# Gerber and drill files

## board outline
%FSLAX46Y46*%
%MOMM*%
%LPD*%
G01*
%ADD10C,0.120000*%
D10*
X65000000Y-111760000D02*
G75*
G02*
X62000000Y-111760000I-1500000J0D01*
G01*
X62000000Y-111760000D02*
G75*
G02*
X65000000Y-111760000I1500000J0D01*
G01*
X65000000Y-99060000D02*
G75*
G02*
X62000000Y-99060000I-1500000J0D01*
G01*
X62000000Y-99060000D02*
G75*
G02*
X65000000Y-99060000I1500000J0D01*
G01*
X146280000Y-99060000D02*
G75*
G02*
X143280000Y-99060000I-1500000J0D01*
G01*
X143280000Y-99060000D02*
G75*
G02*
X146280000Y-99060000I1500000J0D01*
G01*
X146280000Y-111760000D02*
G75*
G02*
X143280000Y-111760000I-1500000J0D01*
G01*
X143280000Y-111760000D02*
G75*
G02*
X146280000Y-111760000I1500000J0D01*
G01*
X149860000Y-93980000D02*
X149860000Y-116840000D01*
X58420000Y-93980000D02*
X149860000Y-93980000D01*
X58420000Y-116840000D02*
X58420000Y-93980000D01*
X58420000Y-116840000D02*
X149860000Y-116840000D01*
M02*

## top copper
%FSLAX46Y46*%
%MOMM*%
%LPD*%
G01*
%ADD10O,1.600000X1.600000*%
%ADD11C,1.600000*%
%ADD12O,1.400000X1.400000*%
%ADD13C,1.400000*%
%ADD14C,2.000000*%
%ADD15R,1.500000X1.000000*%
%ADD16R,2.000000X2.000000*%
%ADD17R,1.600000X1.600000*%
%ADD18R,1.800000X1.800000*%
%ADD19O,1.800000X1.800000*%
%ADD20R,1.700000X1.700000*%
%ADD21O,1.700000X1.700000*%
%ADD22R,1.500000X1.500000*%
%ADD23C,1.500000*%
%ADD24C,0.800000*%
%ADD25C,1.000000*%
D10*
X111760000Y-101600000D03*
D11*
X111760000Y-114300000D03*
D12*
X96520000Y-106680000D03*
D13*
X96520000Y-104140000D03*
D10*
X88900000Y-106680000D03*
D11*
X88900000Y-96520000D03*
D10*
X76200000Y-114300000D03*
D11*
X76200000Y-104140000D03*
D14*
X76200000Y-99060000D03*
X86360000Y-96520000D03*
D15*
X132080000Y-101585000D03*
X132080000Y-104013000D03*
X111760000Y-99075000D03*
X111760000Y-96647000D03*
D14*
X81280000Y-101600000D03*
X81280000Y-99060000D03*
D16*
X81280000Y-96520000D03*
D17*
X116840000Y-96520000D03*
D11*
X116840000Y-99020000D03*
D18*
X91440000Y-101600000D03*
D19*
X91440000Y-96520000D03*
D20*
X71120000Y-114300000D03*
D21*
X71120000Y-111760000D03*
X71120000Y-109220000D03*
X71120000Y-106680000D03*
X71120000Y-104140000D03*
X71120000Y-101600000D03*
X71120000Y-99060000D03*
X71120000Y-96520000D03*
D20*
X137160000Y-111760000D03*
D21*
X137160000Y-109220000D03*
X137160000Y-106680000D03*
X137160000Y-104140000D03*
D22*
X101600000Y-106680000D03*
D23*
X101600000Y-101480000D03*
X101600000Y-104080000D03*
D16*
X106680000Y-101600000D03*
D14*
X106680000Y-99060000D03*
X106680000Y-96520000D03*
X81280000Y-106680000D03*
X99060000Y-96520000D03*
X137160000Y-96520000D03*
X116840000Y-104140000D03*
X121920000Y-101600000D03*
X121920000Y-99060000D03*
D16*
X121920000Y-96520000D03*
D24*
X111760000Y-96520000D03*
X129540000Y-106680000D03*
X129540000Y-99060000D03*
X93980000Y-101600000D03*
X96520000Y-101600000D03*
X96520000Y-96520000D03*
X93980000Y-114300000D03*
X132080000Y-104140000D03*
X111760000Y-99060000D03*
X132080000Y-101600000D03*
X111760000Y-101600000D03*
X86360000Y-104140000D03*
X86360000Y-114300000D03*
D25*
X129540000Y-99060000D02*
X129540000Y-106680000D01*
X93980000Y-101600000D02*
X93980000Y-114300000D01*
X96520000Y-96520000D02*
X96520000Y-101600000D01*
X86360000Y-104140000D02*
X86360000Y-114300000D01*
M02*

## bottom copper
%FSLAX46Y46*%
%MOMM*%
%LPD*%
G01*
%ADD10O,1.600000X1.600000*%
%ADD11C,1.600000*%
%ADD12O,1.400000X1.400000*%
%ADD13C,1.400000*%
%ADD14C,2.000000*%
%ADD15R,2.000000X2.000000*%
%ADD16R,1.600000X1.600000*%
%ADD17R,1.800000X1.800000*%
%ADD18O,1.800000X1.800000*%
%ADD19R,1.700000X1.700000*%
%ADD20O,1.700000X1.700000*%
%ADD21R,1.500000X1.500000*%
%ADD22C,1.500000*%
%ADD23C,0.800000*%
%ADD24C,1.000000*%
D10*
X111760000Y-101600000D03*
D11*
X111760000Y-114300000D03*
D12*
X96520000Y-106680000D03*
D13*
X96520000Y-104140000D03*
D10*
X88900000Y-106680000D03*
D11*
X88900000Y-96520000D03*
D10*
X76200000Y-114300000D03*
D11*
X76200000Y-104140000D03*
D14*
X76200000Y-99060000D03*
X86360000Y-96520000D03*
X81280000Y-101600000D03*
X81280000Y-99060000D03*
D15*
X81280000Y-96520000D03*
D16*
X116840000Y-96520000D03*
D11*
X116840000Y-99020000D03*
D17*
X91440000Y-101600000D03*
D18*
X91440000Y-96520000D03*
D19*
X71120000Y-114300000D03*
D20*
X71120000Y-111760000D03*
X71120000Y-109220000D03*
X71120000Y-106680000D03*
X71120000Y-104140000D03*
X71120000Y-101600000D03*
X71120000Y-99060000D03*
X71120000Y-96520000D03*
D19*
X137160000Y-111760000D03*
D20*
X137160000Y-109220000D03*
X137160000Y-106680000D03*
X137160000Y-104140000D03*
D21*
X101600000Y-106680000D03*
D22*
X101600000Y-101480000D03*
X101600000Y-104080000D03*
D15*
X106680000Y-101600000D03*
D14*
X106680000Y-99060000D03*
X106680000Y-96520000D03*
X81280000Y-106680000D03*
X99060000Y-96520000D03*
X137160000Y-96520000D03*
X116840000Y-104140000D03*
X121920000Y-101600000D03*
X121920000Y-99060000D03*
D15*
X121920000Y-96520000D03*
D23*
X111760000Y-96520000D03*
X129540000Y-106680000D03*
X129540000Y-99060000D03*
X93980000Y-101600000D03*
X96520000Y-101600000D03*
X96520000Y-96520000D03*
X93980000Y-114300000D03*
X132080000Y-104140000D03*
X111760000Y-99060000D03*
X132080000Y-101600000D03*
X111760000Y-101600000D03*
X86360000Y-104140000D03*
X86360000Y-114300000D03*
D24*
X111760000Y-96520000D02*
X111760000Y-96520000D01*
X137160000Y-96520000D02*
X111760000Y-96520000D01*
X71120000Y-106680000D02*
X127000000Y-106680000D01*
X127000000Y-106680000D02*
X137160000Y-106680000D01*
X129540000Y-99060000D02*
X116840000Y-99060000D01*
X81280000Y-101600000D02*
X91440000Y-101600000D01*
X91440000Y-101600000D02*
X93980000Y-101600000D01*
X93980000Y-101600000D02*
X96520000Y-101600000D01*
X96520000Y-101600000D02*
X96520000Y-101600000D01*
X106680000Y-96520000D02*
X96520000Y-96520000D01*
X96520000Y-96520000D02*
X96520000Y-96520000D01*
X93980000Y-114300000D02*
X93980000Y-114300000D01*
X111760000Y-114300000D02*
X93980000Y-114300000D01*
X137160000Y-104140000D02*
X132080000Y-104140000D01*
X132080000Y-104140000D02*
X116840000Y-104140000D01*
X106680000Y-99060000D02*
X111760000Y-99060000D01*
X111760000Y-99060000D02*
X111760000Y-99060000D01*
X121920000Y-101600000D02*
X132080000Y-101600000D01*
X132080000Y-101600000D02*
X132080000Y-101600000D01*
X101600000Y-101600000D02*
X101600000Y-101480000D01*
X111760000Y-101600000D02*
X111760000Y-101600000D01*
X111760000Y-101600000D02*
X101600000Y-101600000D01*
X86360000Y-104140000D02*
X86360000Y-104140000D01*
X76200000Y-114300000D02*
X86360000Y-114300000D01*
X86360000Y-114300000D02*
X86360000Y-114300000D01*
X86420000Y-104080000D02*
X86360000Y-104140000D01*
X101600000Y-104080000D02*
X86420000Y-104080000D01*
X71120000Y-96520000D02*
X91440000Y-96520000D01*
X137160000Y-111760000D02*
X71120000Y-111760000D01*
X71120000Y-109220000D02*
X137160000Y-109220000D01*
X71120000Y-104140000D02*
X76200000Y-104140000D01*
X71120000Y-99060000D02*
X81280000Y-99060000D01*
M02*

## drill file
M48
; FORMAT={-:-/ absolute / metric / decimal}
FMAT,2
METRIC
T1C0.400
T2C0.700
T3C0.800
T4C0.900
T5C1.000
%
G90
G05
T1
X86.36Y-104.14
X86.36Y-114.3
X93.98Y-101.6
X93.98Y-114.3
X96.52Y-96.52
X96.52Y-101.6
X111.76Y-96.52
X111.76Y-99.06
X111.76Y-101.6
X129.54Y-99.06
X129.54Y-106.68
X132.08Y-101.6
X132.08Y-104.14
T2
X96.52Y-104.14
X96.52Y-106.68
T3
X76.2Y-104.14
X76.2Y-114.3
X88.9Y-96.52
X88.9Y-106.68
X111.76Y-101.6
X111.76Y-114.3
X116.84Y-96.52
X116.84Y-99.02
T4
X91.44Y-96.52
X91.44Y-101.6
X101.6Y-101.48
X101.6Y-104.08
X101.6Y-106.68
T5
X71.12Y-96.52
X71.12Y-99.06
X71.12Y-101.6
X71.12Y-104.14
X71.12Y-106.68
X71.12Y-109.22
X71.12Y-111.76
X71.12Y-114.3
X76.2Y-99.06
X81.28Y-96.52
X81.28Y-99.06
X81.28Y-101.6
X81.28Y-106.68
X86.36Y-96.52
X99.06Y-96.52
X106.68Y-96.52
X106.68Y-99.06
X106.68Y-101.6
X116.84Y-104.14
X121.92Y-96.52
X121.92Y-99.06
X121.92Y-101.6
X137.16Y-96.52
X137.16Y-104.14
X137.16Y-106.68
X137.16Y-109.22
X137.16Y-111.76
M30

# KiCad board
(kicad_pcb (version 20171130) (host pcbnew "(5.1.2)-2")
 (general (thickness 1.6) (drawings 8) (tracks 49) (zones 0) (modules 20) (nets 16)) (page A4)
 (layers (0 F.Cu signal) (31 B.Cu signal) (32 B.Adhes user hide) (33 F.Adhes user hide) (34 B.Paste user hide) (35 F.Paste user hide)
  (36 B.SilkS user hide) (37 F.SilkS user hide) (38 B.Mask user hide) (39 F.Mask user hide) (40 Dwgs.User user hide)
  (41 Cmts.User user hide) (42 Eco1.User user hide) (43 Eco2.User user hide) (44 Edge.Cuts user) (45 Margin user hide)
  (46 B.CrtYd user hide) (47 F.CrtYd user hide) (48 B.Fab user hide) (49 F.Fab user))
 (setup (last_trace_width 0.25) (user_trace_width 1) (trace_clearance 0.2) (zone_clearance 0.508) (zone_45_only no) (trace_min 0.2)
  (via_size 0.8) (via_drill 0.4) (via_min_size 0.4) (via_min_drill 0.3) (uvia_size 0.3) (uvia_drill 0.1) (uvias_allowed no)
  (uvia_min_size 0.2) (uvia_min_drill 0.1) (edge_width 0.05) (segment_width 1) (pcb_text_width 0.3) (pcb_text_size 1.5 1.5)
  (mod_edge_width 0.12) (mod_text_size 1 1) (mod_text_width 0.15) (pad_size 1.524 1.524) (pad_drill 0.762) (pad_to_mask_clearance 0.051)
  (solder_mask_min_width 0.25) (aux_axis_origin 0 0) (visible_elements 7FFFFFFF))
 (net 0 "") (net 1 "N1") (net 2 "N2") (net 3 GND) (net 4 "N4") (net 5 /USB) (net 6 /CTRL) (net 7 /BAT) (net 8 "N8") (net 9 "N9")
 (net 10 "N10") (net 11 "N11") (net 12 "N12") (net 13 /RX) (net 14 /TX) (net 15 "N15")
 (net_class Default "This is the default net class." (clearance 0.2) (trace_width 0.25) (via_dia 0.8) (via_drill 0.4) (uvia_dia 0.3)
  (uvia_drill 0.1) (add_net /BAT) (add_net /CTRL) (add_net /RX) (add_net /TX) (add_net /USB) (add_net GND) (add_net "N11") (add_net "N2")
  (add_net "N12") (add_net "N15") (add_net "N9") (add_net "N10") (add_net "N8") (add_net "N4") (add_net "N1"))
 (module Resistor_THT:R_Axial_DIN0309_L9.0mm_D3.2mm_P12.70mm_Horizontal (layer F.Cu) (at 111.76 114.3 90)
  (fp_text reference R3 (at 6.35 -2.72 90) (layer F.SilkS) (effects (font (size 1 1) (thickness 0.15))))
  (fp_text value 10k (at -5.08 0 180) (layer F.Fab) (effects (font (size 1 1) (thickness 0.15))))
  (pad 2 thru_hole oval (at 12.7 0 90) (size 1.6 1.6) (drill 0.8) (layers *.Cu *.Mask) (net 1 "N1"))
  (pad 1 thru_hole circle (at 0 0 90) (size 1.6 1.6) (drill 0.8) (layers *.Cu *.Mask) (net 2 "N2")))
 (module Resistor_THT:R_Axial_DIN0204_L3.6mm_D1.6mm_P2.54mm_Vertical (layer F.Cu) (at 96.52 104.14 270)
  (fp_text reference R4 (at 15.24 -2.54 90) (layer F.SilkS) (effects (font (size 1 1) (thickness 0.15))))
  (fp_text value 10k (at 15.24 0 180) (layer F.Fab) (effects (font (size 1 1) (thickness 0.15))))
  (pad 2 thru_hole oval (at 2.54 0 270) (size 1.4 1.4) (drill 0.7) (layers *.Cu *.Mask) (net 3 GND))
  (pad 1 thru_hole circle (at 0 0 270) (size 1.4 1.4) (drill 0.7) (layers *.Cu *.Mask) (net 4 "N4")))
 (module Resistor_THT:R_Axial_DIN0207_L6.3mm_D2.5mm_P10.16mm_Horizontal (layer F.Cu) (at 88.9 96.52 270)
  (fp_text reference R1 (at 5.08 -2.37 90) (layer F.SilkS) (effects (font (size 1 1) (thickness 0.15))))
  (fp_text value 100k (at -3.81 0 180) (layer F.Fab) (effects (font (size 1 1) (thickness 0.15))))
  (pad 2 thru_hole oval (at 10.16 0 270) (size 1.6 1.6) (drill 0.8) (layers *.Cu *.Mask) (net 3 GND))
  (pad 1 thru_hole circle (at 0 0 270) (size 1.6 1.6) (drill 0.8) (layers *.Cu *.Mask) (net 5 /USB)))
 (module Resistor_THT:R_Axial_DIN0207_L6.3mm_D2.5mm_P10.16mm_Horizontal (layer F.Cu) (at 76.2 104.14 270)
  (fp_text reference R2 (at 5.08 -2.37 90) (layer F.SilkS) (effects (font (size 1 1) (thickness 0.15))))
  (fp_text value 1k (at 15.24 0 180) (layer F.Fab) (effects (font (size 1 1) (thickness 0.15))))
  (pad 2 thru_hole oval (at 10.16 0 270) (size 1.6 1.6) (drill 0.8) (layers *.Cu *.Mask) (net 4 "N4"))
  (pad 1 thru_hole circle (at 0 0 270) (size 1.6 1.6) (drill 0.8) (layers *.Cu *.Mask) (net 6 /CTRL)))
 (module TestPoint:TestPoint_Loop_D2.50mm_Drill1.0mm (layer F.Cu) (at 76.2 99.06)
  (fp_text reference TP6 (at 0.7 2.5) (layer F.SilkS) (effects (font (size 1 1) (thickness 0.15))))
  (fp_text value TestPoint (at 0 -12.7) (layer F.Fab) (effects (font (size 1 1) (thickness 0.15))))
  (pad 1 thru_hole circle (at 0 0) (size 2 2) (drill 1) (layers *.Cu *.Mask) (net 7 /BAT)))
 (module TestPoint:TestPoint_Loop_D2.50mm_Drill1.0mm (layer F.Cu) (at 86.36 96.52)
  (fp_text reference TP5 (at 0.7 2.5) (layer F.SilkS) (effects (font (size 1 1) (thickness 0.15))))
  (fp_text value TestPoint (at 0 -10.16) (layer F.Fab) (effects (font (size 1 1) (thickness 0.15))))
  (pad 1 thru_hole circle (at 0 0) (size 2 2) (drill 1) (layers *.Cu *.Mask) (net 5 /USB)))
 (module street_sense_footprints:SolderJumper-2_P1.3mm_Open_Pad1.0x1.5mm (layer F.Cu) (at 132.08 101.6 270)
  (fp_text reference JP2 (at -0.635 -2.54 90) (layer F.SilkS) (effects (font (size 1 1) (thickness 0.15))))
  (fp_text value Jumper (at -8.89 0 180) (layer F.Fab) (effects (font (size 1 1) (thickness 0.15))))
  (pad 1 smd rect (at -0.015 0 270) (size 1 1.5) (layers F.Cu F.Mask) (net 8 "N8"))
  (pad 2 smd rect (at 2.413 0 270) (size 1 1.5) (layers F.Cu F.Mask) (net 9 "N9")))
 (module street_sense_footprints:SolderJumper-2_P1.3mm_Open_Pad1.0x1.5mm (layer F.Cu) (at 111.76 99.06 90)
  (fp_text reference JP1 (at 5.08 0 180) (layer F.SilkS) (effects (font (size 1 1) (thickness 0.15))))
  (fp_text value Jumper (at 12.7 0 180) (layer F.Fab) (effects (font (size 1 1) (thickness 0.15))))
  (pad 1 smd rect (at -0.015 0 90) (size 1 1.5) (layers F.Cu F.Mask) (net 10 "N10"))
  (pad 2 smd rect (at 2.413 0 90) (size 1 1.5) (layers F.Cu F.Mask) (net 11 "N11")))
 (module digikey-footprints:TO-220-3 (layer F.Cu) (at 81.28 96.52 270)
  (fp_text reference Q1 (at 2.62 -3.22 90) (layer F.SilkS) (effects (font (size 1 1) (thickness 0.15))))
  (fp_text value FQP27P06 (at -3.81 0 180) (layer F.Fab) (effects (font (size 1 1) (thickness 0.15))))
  (pad 3 thru_hole circle (at 5.08 0 270) (size 2 2) (drill 1) (layers *.Cu *.Mask) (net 2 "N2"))
  (pad 2 thru_hole circle (at 2.54 0 270) (size 2 2) (drill 1) (layers *.Cu *.Mask) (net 7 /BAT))
  (pad 1 thru_hole rect (at 0 0 270) (size 2 2) (drill 1) (layers *.Cu *.Mask) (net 5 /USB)))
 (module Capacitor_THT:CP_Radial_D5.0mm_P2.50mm (layer F.Cu) (at 116.84 96.52 270)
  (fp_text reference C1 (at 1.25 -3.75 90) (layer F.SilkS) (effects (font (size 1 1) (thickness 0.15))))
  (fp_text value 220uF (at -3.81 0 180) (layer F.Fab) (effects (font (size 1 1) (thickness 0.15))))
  (pad 1 thru_hole rect (at 0 0 270) (size 1.6 1.6) (drill 0.8) (layers *.Cu *.Mask) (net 11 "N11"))
  (pad 2 thru_hole circle (at 2.5 0 270) (size 1.6 1.6) (drill 0.8) (layers *.Cu *.Mask) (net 3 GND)))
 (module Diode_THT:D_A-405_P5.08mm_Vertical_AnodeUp (layer F.Cu) (at 91.44 101.6 90)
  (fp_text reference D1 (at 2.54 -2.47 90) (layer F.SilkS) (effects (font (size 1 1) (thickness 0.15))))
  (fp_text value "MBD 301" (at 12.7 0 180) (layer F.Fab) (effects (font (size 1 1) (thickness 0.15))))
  (pad 1 thru_hole rect (at 0 0 90) (size 1.8 1.8) (drill 0.9) (layers *.Cu *.Mask) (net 2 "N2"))
  (pad 2 thru_hole oval (at 5.08 0 90) (size 1.8 1.8) (drill 0.9) (layers *.Cu *.Mask) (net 5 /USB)))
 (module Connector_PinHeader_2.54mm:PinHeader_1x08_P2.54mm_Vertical (layer F.Cu) (at 71.12 114.3 180)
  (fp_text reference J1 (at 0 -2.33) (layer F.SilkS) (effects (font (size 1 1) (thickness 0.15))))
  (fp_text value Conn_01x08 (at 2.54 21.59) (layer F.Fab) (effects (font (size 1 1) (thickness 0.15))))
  (pad 1 thru_hole rect (at 0 0 180) (size 1.7 1.7) (drill 1) (layers *.Cu *.Mask) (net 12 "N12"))
  (pad 2 thru_hole oval (at 0 2.54 180) (size 1.7 1.7) (drill 1) (layers *.Cu *.Mask) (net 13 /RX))
  (pad 3 thru_hole oval (at 0 5.08 180) (size 1.7 1.7) (drill 1) (layers *.Cu *.Mask) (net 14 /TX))
  (pad 4 thru_hole oval (at 0 7.62 180) (size 1.7 1.7) (drill 1) (layers *.Cu *.Mask) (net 3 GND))
  (pad 5 thru_hole oval (at 0 10.16 180) (size 1.7 1.7) (drill 1) (layers *.Cu *.Mask) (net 6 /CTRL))
  (pad 6 thru_hole oval (at 0 12.7 180) (size 1.7 1.7) (drill 1) (layers *.Cu *.Mask) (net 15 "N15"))
  (pad 7 thru_hole oval (at 0 15.24 180) (size 1.7 1.7) (drill 1) (layers *.Cu *.Mask) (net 7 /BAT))
  (pad 8 thru_hole oval (at 0 17.78 180) (size 1.7 1.7) (drill 1) (layers *.Cu *.Mask) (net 5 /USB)))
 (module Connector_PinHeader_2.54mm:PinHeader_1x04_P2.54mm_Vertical (layer F.Cu) (at 137.16 111.76 180)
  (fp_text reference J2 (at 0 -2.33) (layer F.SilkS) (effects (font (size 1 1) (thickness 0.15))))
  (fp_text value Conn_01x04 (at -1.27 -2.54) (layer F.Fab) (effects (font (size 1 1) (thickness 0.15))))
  (pad 1 thru_hole rect (at 0 0 180) (size 1.7 1.7) (drill 1) (layers *.Cu *.Mask) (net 13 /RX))
  (pad 2 thru_hole oval (at 0 2.54 180) (size 1.7 1.7) (drill 1) (layers *.Cu *.Mask) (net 14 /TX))
  (pad 3 thru_hole oval (at 0 5.08 180) (size 1.7 1.7) (drill 1) (layers *.Cu *.Mask) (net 3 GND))
  (pad 4 thru_hole oval (at 0 7.62 180) (size 1.7 1.7) (drill 1) (layers *.Cu *.Mask) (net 9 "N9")))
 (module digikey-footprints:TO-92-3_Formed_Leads (layer F.Cu) (at 101.6 106.68 90)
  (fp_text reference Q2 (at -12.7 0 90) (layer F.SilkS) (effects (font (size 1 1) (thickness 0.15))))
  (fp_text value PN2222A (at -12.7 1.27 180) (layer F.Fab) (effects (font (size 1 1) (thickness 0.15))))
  (pad 1 thru_hole rect (at 0 0 270) (size 1.5 1.5) (drill 0.9) (layers *.Cu *.Mask) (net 3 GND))
  (pad 3 thru_hole circle (at 5.2 0 270) (size 1.5 1.5) (drill 0.9) (layers *.Cu *.Mask) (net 1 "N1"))
  (pad 2 thru_hole circle (at 2.6 0 270) (size 1.5 1.5) (drill 0.9) (layers *.Cu *.Mask) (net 4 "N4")))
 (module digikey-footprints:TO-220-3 (layer F.Cu) (at 106.68 101.6 90)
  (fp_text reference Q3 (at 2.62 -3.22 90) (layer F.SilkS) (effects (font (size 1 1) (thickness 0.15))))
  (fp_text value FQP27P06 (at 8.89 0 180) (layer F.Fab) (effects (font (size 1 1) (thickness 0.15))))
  (pad 1 thru_hole rect (at 0 0 90) (size 2 2) (drill 1) (layers *.Cu *.Mask) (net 1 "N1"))
  (pad 2 thru_hole circle (at 2.54 0 90) (size 2 2) (drill 1) (layers *.Cu *.Mask) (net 10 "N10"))
  (pad 3 thru_hole circle (at 5.08 0 90) (size 2 2) (drill 1) (layers *.Cu *.Mask) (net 2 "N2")))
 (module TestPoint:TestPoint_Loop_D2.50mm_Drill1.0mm (layer F.Cu) (at 81.28 106.68)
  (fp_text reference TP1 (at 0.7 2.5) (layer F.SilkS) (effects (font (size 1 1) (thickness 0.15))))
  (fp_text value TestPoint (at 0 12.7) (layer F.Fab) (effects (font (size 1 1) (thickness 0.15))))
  (pad 1 thru_hole circle (at 0 0) (size 2 2) (drill 1) (layers *.Cu *.Mask) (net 3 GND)))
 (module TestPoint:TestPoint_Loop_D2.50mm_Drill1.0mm (layer F.Cu) (at 99.06 96.52)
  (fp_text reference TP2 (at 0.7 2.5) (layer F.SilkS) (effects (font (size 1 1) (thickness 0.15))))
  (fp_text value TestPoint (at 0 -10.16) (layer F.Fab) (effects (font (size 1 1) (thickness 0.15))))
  (pad 1 thru_hole circle (at 0 0) (size 2 2) (drill 1) (layers *.Cu *.Mask) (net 2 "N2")))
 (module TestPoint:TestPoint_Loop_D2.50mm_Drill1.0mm (layer F.Cu) (at 137.16 96.52)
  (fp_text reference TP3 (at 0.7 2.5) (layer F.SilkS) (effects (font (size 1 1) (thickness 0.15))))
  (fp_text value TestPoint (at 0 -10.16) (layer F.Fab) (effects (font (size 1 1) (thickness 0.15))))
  (pad 1 thru_hole circle (at 0 0) (size 2 2) (drill 1) (layers *.Cu *.Mask) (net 11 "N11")))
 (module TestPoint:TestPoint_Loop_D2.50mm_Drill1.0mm (layer F.Cu) (at 116.84 104.14)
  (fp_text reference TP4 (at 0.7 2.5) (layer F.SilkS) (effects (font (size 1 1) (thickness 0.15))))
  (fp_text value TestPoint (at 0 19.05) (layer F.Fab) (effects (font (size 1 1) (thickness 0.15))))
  (pad 1 thru_hole circle (at 0 0) (size 2 2) (drill 1) (layers *.Cu *.Mask) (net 9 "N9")))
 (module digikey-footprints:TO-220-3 (layer F.Cu) (at 121.92 96.52 270)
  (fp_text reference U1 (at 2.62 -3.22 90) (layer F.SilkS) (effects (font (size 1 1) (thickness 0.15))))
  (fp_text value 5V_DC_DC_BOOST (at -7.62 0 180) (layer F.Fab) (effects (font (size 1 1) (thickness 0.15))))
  (pad 3 thru_hole circle (at 5.08 0 270) (size 2 2) (drill 1) (layers *.Cu *.Mask) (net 8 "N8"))
  (pad 2 thru_hole circle (at 2.54 0 270) (size 2 2) (drill 1) (layers *.Cu *.Mask) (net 3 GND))
  (pad 1 thru_hole rect (at 0 0 270) (size 2 2) (drill 1) (layers *.Cu *.Mask) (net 11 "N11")))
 (gr_circle (center 63.5 111.76) (end 65 111.76) (layer Edge.Cuts) (width 0.12))
 (gr_circle (center 63.5 99.06) (end 65 99.06) (layer Edge.Cuts) (width 0.12))
 (gr_circle (center 144.78 99.06) (end 146.28 99.06) (layer Edge.Cuts) (width 0.12))
 (gr_circle (center 144.78 111.76) (end 146.28 111.76) (layer Edge.Cuts) (width 0.12))
 (gr_line (start 149.86 93.98) (end 149.86 116.84) (layer Edge.Cuts) (width 0.12))
 (gr_line (start 58.42 93.98) (end 149.86 93.98) (layer Edge.Cuts) (width 0.12))
 (gr_line (start 58.42 116.84) (end 58.42 93.98) (layer Edge.Cuts) (width 0.12))
 (gr_line (start 58.42 116.84) (end 149.86 116.84) (layer Edge.Cuts) (width 0.12))
 (segment (start 111.76 96.52) (end 111.76 96.52) (width 1) (layer B.Cu) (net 11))
 (via (at 111.76 96.52) (size 0.8) (drill 0.4) (layers F.Cu B.Cu) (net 11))
 (segment (start 137.16 96.52) (end 111.76 96.52) (width 1) (layer B.Cu) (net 11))
 (segment (start 71.12 106.68) (end 127 106.68) (width 1) (layer B.Cu) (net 3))
 (segment (start 127 106.68) (end 137.16 106.68) (width 1) (layer B.Cu) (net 3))
 (via (at 129.54 106.68) (size 0.8) (drill 0.4) (layers F.Cu B.Cu) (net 3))
 (segment (start 129.54 99.06) (end 129.54 106.68) (width 1) (layer F.Cu) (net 3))
 (via (at 129.54 99.06) (size 0.8) (drill 0.4) (layers F.Cu B.Cu) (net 3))
 (segment (start 129.54 99.06) (end 116.84 99.06) (width 1) (layer B.Cu) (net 3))
 (segment (start 81.28 101.6) (end 91.44 101.6) (width 1) (layer B.Cu) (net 2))
 (segment (start 91.44 101.6) (end 93.98 101.6) (width 1) (layer B.Cu) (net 2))
 (segment (start 93.98 101.6) (end 96.52 101.6) (width 1) (layer B.Cu) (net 2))
 (via (at 93.98 101.6) (size 0.8) (drill 0.4) (layers F.Cu B.Cu) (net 2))
 (segment (start 93.98 101.6) (end 93.98 114.3) (width 1) (layer F.Cu) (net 2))
 (segment (start 96.52 101.6) (end 96.52 101.6) (width 1) (layer B.Cu) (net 2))
 (via (at 96.52 101.6) (size 0.8) (drill 0.4) (layers F.Cu B.Cu) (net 2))
 (segment (start 106.68 96.52) (end 96.52 96.52) (width 1) (layer B.Cu) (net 2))
 (segment (start 96.52 96.52) (end 96.52 96.52) (width 1) (layer B.Cu) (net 2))
 (via (at 96.52 96.52) (size 0.8) (drill 0.4) (layers F.Cu B.Cu) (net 2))
 (segment (start 96.52 96.52) (end 96.52 101.6) (width 1) (layer F.Cu) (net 2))
 (segment (start 93.98 114.3) (end 93.98 114.3) (width 1) (layer B.Cu) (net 2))
 (via (at 93.98 114.3) (size 0.8) (drill 0.4) (layers F.Cu B.Cu) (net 2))
 (segment (start 111.76 114.3) (end 93.98 114.3) (width 1) (layer B.Cu) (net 2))
 (segment (start 137.16 104.14) (end 132.08 104.14) (width 1) (layer B.Cu) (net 9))
 (segment (start 132.08 104.14) (end 116.84 104.14) (width 1) (layer B.Cu) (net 9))
 (via (at 132.08 104.14) (size 0.8) (drill 0.4) (layers F.Cu B.Cu) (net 9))
 (segment (start 106.68 99.06) (end 111.76 99.06) (width 1) (layer B.Cu) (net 10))
 (segment (start 111.76 99.06) (end 111.76 99.06) (width 1) (layer B.Cu) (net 10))
 (via (at 111.76 99.06) (size 0.8) (drill 0.4) (layers F.Cu B.Cu) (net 10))
 (segment (start 121.92 101.6) (end 132.08 101.6) (width 1) (layer B.Cu) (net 8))
 (segment (start 132.08 101.6) (end 132.08 101.6) (width 1) (layer B.Cu) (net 8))
 (via (at 132.08 101.6) (size 0.8) (drill 0.4) (layers F.Cu B.Cu) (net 8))
 (segment (start 101.6 101.6) (end 101.6 101.48) (width 1) (layer B.Cu) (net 1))
 (segment (start 111.76 101.6) (end 111.76 101.6) (width 1) (layer B.Cu) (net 1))
 (segment (start 111.76 101.6) (end 101.6 101.6) (width 1) (layer B.Cu) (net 1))
 (via (at 111.76 101.6) (size 0.8) (drill 0.4) (layers F.Cu B.Cu) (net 1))
 (segment (start 86.36 104.14) (end 86.36 104.14) (width 1) (layer B.Cu) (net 4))
 (segment (start 76.2 114.3) (end 86.36 114.3) (width 1) (layer B.Cu) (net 4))
 (via (at 86.36 104.14) (size 0.8) (drill 0.4) (layers F.Cu B.Cu) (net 4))
 (segment (start 86.36 114.3) (end 86.36 114.3) (width 1) (layer B.Cu) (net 4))
 (via (at 86.36 114.3) (size 0.8) (drill 0.4) (layers F.Cu B.Cu) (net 4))
 (segment (start 86.36 104.14) (end 86.36 114.3) (width 1) (layer F.Cu) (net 4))
 (segment (start 86.42 104.08) (end 86.36 104.14) (width 1) (layer B.Cu) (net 4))
 (segment (start 101.6 104.08) (end 86.42 104.08) (width 1) (layer B.Cu) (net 4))
 (segment (start 71.12 96.52) (end 91.44 96.52) (width 1) (layer B.Cu) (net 5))
 (segment (start 137.16 111.76) (end 71.12 111.76) (width 1) (layer B.Cu) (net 13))
 (segment (start 71.12 109.22) (end 137.16 109.22) (width 1) (layer B.Cu) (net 14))
 (segment (start 71.12 104.14) (end 76.2 104.14) (width 1) (layer B.Cu) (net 6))
 (segment (start 71.12 99.06) (end 81.28 99.06) (width 1) (layer B.Cu) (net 7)))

